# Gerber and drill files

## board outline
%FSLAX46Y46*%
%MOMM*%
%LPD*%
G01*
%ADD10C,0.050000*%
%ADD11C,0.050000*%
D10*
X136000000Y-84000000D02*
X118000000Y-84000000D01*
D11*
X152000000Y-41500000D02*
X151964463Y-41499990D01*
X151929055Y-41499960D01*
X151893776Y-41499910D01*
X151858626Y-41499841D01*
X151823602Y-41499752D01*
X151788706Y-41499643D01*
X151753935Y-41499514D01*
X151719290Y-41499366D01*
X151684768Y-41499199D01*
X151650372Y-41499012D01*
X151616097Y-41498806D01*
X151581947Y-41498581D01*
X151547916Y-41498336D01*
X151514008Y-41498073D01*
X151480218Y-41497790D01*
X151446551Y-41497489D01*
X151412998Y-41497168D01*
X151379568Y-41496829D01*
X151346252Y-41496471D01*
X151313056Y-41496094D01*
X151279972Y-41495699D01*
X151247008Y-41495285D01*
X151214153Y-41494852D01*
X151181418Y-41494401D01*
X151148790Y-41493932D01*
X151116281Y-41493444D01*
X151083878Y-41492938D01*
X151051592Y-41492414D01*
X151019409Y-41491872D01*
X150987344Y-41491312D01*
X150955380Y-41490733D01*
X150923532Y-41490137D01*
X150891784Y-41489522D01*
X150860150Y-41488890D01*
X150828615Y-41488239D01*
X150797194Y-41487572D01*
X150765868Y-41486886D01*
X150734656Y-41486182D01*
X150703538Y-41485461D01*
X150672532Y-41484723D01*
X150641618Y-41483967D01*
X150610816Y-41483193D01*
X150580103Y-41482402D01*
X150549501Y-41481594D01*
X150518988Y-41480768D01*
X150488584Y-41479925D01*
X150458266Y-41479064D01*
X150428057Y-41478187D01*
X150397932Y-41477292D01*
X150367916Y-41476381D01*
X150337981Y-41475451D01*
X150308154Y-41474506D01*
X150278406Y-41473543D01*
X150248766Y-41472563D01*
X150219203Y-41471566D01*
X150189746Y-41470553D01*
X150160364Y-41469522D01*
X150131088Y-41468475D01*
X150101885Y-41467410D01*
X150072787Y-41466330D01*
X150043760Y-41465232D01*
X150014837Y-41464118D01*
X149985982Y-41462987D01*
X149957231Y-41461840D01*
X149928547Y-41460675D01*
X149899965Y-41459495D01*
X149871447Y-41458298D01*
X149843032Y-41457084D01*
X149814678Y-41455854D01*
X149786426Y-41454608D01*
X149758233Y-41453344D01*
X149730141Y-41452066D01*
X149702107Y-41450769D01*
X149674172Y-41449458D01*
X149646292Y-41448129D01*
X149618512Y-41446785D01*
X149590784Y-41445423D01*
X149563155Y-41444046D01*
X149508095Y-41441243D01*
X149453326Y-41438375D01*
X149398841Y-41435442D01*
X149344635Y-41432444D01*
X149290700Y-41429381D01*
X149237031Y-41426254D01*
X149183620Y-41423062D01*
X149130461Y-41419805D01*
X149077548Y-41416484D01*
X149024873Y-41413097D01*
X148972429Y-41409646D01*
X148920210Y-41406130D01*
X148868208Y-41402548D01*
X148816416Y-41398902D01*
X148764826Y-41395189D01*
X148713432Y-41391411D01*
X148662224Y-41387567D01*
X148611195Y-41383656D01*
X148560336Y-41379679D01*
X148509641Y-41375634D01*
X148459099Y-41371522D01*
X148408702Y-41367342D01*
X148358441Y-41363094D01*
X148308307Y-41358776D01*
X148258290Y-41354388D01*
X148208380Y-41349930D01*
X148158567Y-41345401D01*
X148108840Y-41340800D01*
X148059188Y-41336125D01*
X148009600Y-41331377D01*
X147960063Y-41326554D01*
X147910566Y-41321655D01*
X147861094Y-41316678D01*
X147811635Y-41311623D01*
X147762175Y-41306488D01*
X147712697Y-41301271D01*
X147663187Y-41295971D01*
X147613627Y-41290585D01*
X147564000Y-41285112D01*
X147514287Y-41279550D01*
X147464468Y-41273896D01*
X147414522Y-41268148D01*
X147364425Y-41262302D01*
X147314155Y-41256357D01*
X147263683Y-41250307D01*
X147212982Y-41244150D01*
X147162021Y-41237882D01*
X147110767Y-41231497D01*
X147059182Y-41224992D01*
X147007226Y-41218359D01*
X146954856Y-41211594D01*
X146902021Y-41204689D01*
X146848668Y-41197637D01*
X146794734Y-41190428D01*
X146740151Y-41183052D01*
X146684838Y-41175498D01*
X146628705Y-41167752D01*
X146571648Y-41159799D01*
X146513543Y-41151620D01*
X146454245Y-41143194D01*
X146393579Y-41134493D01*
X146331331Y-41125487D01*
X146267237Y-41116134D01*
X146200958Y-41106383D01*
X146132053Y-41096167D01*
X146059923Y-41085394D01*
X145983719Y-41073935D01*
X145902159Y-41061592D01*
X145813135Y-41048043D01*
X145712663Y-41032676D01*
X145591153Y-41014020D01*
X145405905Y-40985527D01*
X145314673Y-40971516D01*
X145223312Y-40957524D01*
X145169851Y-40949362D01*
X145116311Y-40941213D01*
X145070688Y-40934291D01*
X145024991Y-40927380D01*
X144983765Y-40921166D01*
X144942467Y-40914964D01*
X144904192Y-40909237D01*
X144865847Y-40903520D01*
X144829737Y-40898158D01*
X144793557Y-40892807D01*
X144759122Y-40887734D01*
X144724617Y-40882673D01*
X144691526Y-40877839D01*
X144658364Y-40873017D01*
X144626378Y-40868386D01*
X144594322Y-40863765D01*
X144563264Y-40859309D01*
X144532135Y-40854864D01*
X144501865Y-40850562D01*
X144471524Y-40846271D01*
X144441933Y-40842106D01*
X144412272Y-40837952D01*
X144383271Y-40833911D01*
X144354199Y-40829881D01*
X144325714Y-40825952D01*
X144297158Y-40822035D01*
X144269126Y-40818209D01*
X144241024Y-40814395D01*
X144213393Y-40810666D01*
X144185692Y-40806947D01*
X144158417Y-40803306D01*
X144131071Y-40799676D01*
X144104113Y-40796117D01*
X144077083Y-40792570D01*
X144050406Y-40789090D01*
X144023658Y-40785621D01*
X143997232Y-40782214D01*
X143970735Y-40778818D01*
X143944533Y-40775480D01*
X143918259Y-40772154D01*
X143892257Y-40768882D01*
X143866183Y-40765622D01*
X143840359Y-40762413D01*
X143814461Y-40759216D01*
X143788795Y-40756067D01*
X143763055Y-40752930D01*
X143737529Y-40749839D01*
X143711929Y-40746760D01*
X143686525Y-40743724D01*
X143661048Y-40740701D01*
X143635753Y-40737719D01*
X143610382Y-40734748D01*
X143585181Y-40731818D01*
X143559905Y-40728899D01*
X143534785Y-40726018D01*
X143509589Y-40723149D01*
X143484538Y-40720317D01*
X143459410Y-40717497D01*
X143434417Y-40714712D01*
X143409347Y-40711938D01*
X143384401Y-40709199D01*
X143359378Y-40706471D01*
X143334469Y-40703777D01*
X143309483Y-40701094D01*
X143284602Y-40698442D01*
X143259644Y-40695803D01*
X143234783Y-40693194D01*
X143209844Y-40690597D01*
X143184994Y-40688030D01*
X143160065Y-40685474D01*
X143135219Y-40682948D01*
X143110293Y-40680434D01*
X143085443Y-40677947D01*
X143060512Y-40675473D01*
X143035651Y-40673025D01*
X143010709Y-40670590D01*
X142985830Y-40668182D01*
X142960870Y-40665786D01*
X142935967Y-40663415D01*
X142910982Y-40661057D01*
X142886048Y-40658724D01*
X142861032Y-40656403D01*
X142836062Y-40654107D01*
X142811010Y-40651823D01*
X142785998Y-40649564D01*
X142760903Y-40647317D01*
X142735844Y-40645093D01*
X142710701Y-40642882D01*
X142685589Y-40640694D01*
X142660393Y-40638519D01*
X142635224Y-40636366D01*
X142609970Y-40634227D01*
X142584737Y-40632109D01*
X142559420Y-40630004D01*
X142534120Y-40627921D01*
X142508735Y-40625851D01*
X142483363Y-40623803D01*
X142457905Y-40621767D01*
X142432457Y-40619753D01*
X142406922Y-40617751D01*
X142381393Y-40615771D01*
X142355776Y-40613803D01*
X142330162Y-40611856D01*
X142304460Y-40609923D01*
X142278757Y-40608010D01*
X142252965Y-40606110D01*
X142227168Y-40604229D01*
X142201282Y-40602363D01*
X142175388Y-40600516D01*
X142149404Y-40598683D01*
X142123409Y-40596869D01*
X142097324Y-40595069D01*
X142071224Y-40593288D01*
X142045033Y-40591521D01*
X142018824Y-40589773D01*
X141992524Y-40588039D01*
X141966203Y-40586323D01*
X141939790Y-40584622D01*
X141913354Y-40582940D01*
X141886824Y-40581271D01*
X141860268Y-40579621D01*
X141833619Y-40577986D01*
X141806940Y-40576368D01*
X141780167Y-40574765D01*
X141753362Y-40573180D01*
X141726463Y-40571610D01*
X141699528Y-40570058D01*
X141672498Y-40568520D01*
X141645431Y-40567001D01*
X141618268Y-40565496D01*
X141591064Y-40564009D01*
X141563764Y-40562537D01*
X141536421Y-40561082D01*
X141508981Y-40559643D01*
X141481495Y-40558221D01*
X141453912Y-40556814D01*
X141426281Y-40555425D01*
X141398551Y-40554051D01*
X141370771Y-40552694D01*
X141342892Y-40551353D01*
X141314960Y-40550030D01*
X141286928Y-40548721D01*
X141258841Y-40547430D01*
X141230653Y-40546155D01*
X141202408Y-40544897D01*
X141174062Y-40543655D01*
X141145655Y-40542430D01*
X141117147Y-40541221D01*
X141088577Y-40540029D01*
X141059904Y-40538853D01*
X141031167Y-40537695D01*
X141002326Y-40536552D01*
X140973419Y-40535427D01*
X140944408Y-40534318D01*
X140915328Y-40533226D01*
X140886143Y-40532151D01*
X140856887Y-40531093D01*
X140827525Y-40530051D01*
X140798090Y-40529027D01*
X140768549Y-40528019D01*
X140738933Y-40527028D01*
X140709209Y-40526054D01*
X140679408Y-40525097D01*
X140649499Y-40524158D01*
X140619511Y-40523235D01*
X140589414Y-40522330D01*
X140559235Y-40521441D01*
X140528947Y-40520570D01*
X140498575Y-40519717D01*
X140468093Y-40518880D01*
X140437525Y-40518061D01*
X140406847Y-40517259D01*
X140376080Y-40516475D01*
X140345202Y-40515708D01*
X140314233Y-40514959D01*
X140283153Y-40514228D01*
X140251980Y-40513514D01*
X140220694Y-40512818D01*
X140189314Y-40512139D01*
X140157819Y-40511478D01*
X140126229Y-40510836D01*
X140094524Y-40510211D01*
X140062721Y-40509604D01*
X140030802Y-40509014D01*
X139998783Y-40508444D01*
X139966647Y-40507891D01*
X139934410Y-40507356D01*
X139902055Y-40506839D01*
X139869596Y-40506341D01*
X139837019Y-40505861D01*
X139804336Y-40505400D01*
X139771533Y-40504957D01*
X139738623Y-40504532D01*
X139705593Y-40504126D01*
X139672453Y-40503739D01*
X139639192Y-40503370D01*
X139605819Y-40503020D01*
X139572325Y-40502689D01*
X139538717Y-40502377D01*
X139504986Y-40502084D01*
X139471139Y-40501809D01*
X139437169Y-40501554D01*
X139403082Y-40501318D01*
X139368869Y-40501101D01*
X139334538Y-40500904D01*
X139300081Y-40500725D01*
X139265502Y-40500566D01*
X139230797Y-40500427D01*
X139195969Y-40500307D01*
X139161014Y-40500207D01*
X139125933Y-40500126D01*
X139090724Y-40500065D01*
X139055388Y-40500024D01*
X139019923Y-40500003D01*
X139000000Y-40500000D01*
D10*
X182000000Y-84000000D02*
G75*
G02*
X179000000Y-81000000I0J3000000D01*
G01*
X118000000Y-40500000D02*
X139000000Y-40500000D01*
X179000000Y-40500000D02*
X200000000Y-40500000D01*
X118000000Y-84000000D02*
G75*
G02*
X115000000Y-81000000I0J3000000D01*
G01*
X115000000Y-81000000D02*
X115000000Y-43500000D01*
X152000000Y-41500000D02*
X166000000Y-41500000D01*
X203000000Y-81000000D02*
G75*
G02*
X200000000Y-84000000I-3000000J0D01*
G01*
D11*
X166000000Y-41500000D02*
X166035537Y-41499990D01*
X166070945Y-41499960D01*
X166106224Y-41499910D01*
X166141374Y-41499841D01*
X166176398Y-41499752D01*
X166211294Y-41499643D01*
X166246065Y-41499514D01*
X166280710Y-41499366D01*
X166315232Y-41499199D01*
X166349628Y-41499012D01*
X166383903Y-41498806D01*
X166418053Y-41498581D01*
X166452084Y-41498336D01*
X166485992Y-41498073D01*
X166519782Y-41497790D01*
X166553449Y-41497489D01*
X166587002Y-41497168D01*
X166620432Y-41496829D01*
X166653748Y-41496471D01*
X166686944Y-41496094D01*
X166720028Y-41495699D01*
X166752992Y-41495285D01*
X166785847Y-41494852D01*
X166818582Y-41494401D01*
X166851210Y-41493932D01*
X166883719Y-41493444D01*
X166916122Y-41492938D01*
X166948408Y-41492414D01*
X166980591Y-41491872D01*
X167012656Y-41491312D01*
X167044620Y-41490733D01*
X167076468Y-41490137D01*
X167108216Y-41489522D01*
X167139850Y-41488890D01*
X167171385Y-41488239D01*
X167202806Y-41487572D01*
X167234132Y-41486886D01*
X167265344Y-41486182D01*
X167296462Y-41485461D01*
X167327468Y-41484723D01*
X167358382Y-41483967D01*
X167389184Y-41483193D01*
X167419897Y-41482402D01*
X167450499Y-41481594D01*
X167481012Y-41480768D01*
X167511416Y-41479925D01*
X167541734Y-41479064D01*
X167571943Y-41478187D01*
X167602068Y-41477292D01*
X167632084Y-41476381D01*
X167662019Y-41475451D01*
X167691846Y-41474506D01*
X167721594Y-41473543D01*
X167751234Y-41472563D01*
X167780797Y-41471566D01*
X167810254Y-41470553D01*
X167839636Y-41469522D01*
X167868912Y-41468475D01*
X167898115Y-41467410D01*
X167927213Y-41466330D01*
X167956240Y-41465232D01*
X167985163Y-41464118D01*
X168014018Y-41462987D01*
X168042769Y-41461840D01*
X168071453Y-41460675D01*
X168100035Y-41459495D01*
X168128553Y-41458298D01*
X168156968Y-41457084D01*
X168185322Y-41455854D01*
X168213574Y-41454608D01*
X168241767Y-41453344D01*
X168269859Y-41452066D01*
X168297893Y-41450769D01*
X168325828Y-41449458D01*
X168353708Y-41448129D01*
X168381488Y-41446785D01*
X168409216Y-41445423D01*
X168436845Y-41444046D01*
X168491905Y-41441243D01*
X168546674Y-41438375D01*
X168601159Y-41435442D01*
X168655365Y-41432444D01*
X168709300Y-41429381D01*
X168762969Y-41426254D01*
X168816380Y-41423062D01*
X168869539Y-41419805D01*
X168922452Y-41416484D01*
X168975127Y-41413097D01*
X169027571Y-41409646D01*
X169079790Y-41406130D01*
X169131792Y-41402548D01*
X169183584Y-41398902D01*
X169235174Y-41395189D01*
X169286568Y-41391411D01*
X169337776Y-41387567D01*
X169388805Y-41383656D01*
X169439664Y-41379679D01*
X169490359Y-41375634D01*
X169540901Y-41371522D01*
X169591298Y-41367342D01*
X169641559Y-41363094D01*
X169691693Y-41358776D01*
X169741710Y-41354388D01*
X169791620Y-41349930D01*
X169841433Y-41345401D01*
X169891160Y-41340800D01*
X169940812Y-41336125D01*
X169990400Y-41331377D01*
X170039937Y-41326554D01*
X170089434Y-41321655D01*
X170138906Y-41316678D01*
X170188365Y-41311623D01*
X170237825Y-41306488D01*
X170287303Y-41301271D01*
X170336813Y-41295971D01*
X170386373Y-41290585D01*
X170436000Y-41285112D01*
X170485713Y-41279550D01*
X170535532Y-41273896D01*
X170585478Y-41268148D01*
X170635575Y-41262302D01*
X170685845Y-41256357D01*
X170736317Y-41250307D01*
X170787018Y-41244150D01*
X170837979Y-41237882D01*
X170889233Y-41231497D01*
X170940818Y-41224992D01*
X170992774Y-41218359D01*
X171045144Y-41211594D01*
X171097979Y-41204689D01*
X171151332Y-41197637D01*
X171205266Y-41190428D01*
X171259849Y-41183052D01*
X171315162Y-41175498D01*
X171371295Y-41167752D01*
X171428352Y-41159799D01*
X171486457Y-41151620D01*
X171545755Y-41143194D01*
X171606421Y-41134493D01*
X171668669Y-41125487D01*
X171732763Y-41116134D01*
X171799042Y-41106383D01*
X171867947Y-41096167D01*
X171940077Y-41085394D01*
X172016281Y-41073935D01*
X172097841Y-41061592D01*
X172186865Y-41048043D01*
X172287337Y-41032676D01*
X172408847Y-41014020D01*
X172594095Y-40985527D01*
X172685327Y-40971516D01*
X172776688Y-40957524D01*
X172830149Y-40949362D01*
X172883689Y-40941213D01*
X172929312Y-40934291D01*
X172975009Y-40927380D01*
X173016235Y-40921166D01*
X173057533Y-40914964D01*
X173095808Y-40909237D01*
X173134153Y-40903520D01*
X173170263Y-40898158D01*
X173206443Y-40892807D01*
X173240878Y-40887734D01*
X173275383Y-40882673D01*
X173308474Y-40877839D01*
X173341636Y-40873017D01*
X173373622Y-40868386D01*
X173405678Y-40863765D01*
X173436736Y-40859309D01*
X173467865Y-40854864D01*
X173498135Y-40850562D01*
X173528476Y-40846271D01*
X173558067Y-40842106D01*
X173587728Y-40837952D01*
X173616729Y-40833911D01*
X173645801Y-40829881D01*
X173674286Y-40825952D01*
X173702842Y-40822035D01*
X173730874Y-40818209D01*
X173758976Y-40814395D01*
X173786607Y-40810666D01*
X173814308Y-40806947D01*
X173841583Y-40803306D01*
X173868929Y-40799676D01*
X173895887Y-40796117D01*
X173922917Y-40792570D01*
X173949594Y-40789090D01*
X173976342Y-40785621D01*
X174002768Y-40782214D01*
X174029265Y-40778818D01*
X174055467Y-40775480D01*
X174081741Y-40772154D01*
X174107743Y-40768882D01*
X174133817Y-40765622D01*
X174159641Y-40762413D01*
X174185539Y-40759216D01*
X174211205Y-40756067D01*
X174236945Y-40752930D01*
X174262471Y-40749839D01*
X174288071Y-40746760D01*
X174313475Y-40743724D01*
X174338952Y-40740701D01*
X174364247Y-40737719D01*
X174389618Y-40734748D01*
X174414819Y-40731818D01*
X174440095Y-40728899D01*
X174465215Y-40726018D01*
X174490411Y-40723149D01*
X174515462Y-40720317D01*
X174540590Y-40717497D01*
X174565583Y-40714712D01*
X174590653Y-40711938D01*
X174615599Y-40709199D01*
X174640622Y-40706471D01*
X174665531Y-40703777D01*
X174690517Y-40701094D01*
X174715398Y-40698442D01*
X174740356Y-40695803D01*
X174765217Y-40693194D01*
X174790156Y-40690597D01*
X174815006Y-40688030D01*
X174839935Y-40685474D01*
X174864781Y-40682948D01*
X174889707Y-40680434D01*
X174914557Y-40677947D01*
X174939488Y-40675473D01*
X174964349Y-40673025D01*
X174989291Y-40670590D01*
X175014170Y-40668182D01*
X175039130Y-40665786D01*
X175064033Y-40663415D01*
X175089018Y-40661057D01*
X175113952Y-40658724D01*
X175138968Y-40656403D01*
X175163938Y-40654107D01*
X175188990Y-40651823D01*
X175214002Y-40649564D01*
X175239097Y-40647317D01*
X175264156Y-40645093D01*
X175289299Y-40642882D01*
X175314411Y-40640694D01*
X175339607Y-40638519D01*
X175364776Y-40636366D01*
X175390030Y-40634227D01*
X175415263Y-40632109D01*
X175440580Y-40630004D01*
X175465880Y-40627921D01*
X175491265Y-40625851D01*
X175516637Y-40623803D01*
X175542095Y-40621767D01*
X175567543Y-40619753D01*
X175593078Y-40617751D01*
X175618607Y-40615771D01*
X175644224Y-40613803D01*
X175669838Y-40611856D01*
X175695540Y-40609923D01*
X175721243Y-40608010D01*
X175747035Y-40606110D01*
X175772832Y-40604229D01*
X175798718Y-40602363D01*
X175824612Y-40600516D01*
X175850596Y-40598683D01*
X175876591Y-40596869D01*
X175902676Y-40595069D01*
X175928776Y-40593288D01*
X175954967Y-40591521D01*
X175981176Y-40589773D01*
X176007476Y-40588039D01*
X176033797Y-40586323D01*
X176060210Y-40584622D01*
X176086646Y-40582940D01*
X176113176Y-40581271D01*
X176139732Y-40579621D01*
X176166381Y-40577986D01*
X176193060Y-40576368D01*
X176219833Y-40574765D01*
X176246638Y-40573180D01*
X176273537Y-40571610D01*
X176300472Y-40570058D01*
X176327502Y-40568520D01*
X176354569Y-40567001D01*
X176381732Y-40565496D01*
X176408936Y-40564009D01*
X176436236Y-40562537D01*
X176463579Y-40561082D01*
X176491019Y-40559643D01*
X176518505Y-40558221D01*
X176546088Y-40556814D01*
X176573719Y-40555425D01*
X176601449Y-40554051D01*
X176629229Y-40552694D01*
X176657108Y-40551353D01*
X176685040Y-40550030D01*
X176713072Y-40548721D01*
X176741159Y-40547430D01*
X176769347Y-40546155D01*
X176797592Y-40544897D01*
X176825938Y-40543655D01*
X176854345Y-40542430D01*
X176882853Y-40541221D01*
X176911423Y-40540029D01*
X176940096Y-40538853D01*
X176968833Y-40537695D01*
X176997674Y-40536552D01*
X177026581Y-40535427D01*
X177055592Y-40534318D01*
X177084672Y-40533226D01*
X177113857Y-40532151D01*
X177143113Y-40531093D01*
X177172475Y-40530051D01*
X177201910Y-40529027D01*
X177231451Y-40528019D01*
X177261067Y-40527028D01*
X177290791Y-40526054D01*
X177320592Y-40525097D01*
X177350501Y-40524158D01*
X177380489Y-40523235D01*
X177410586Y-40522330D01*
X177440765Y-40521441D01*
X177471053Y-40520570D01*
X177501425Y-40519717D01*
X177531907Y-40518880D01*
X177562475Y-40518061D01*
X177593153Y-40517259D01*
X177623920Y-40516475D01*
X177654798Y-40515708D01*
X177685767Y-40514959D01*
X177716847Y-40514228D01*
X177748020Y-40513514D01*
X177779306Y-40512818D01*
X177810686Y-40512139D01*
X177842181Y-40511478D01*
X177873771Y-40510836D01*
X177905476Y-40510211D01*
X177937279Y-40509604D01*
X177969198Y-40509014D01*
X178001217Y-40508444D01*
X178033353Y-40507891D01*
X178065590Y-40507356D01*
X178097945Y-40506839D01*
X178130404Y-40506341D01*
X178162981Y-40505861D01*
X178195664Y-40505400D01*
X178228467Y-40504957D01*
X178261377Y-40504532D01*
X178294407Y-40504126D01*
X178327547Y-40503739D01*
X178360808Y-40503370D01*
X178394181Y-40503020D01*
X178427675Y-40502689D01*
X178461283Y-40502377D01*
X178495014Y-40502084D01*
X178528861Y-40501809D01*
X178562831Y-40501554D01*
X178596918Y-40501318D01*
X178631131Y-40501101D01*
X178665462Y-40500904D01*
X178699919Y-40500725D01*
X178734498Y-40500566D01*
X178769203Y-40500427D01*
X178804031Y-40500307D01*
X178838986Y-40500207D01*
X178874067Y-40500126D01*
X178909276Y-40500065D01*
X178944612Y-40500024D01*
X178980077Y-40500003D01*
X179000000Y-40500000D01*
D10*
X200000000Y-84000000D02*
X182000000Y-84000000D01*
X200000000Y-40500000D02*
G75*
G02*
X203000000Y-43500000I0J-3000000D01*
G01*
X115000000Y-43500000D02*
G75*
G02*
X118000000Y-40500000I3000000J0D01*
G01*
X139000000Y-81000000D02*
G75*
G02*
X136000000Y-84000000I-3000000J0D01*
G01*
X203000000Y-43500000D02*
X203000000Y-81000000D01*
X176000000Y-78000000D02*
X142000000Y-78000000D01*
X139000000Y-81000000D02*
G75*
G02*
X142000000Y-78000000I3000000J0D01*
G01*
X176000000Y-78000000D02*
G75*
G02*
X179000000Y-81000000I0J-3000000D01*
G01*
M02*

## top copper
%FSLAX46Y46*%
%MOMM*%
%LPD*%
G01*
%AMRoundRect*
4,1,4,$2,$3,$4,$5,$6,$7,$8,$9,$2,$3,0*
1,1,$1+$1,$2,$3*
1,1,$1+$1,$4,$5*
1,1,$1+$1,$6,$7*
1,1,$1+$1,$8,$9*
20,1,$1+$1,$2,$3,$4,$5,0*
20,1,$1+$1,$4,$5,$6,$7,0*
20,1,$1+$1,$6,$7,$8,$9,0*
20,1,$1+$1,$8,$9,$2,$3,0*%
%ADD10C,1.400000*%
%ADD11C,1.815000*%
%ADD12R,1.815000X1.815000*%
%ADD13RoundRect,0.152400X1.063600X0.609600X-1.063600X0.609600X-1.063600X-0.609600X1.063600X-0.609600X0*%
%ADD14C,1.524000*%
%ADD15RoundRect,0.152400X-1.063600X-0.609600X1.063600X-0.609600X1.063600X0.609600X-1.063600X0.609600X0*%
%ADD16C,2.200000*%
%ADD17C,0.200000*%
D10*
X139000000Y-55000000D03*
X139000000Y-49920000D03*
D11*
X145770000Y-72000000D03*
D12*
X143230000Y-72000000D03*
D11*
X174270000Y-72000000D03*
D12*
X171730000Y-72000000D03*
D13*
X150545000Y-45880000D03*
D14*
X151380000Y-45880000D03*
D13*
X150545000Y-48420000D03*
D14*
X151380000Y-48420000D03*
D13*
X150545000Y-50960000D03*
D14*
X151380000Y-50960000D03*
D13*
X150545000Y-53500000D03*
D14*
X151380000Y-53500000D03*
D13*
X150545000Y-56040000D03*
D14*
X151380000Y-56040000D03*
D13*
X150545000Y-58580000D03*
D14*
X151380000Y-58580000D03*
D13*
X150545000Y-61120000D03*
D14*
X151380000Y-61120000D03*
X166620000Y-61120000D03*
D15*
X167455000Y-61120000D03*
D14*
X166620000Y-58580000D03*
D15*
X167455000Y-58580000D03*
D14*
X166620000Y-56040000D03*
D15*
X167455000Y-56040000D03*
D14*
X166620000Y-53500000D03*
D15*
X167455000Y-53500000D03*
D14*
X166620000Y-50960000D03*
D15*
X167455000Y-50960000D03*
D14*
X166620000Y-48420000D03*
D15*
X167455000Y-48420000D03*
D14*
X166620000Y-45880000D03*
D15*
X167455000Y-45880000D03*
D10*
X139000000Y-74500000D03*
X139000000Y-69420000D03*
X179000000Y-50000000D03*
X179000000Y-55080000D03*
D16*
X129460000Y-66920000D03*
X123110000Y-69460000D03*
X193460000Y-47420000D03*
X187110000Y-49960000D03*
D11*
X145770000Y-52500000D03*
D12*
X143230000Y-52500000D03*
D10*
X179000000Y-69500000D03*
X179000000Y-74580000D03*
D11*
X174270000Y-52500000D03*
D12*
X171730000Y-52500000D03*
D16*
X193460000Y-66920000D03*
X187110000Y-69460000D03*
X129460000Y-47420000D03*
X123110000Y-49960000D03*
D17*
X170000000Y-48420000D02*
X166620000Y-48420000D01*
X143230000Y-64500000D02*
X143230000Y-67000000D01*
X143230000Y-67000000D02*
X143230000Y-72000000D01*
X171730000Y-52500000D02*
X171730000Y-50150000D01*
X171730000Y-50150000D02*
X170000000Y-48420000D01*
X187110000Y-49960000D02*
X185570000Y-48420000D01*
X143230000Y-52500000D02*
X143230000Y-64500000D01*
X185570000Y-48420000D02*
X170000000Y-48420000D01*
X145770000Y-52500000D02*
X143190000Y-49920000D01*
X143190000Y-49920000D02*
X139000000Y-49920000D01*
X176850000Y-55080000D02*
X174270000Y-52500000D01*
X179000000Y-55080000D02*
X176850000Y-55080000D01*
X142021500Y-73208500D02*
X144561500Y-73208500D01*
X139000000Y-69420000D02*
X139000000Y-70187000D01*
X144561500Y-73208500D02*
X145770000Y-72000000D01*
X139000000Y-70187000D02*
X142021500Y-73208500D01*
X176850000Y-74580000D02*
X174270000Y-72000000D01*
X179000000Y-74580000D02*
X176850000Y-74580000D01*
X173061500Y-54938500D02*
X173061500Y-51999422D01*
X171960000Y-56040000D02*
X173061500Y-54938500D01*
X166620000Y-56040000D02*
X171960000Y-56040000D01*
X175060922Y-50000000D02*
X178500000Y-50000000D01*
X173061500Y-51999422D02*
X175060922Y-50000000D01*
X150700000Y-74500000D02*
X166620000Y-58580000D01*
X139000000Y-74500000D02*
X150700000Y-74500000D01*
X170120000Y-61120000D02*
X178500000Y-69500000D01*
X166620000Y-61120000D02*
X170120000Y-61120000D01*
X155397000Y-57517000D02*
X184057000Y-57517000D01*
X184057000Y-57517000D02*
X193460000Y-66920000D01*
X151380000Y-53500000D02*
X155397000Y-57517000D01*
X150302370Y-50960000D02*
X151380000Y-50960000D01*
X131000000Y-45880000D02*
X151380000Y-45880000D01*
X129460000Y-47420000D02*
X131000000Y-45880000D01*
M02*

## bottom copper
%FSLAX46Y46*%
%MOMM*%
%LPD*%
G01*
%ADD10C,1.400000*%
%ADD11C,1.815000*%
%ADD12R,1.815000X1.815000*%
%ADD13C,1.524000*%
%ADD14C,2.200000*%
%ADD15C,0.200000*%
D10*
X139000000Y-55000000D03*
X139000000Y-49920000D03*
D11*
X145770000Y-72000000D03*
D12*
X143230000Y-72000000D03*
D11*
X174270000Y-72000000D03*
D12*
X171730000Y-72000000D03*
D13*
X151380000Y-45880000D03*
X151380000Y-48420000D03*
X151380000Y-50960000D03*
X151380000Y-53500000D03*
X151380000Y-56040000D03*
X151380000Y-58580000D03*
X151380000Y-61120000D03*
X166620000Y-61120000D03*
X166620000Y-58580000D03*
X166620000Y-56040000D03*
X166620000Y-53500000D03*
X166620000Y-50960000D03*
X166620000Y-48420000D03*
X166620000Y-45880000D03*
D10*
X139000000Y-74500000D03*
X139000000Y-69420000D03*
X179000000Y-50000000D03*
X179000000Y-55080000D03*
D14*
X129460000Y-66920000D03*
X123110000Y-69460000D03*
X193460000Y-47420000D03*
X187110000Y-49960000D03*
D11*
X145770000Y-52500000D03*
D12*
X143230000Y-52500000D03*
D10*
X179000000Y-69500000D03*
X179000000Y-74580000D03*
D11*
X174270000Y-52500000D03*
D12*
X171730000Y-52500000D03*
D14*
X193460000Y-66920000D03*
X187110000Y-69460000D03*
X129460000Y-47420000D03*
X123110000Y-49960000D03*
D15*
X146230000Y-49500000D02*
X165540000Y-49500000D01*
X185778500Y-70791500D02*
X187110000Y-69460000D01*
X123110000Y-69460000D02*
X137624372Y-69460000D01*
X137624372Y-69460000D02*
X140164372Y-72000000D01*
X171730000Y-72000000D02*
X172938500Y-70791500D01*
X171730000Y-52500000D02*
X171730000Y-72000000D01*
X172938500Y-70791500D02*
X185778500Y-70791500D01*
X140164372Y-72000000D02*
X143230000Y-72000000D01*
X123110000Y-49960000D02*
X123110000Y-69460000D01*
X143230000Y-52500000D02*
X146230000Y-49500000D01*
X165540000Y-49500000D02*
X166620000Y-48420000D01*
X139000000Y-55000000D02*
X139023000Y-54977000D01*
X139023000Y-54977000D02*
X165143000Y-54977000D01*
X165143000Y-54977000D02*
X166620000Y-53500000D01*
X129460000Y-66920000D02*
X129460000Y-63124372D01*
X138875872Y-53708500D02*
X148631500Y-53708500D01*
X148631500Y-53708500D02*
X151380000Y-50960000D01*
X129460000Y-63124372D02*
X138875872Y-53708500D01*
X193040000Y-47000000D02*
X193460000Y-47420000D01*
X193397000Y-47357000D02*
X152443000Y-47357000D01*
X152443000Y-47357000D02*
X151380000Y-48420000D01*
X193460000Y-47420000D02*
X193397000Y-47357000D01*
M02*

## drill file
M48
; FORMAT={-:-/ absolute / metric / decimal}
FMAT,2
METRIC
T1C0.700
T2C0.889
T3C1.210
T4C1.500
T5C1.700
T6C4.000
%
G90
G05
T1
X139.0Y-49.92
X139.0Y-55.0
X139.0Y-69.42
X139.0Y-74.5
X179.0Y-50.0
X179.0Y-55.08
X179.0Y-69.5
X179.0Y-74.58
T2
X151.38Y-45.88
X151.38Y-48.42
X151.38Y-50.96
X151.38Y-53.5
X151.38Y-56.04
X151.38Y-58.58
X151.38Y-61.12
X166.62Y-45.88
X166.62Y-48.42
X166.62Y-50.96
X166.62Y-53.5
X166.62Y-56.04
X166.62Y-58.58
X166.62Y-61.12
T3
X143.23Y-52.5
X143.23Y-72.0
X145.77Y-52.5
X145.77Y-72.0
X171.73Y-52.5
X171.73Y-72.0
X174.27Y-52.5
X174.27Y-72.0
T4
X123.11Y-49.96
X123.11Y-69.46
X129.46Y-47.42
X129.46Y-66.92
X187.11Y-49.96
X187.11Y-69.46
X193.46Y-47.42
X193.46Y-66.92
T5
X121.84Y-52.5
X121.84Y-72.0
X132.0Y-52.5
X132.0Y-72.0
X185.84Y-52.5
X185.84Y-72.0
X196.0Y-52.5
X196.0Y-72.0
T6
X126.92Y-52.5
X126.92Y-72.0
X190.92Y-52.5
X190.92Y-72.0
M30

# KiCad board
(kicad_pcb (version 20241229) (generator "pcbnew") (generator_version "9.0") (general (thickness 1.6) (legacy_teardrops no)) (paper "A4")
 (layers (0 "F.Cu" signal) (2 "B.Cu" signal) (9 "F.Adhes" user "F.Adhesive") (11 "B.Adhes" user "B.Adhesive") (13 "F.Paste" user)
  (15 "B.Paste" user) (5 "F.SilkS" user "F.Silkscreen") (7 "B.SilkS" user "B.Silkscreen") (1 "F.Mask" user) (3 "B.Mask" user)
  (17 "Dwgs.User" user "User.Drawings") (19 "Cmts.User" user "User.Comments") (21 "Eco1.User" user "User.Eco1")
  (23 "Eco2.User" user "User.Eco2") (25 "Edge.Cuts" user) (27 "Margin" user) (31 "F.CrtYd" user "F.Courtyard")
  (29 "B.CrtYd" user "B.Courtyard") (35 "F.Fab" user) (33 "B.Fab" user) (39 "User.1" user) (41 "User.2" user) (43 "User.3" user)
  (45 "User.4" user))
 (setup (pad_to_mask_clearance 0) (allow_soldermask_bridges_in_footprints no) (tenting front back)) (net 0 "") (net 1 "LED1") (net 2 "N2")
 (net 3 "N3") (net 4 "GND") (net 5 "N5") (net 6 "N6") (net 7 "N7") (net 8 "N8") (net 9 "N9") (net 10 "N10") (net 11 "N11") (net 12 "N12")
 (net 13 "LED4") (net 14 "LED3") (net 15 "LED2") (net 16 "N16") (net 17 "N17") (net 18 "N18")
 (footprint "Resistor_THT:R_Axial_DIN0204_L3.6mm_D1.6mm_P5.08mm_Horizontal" (layer "F.Cu") (at 139 55 90)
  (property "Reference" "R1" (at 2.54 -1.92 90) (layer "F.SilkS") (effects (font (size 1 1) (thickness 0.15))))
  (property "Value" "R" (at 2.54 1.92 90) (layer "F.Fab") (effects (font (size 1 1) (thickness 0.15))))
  (pad "1" thru_hole circle (at 0 0 90) (size 1.4 1.4) (drill 0.7) (layers "*.Cu" "*.Mask") (remove_unused_layers no) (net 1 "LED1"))
  (pad "2" thru_hole circle (at 5.08 0 90) (size 1.4 1.4) (drill 0.7) (layers "*.Cu" "*.Mask") (remove_unused_layers no) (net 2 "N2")))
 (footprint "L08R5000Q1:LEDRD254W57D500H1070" (layer "F.Cu") (at 144.5 72)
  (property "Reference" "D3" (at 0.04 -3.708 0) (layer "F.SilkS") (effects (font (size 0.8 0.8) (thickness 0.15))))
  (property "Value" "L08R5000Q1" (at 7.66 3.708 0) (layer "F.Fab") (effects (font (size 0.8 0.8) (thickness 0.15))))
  (pad "A" thru_hole circle (at 1.27 0) (size 1.815 1.815) (drill 1.21) (layers "*.Cu" "*.Mask") (remove_unused_layers no) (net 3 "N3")
   (solder_mask_margin 0.102))
  (pad "C" thru_hole rect (at -1.27 0) (size 1.815 1.815) (drill 1.21) (layers "*.Cu" "*.Mask") (remove_unused_layers no) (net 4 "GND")
   (solder_mask_margin 0.102)))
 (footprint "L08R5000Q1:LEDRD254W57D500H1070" (layer "F.Cu") (at 173 72)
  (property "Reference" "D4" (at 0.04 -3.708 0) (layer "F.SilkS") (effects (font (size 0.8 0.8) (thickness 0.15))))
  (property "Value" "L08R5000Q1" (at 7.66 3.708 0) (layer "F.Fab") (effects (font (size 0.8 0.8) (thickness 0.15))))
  (pad "A" thru_hole circle (at 1.27 0) (size 1.815 1.815) (drill 1.21) (layers "*.Cu" "*.Mask") (remove_unused_layers no) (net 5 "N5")
   (solder_mask_margin 0.102))
  (pad "C" thru_hole rect (at -1.27 0) (size 1.815 1.815) (drill 1.21) (layers "*.Cu" "*.Mask") (remove_unused_layers no) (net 4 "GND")
   (solder_mask_margin 0.102)))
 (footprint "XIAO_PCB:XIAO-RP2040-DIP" (layer "F.Cu") (at 159 53.5)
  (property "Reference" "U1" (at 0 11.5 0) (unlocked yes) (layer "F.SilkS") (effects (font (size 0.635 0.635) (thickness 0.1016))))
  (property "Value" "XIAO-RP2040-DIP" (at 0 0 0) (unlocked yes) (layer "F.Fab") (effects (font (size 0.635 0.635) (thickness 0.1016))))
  (pad "1" smd roundrect (at -8.455 -7.62 180) (size 2.432 1.524) (layers "F.Cu" "F.Mask") (roundrect_rratio 0.1) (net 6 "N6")
   (thermal_bridge_angle 45))
  (pad "1" thru_hole circle (at -7.62 -7.62 180) (size 1.524 1.524) (drill 0.889) (layers "*.Cu" "*.Mask") (remove_unused_layers no)
   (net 6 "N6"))
  (pad "2" smd roundrect (at -8.455 -5.08 180) (size 2.432 1.524) (layers "F.Cu" "F.Mask") (roundrect_rratio 0.1) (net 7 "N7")
   (thermal_bridge_angle 45))
  (pad "2" thru_hole circle (at -7.62 -5.08 180) (size 1.524 1.524) (drill 0.889) (layers "*.Cu" "*.Mask") (remove_unused_layers no)
   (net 7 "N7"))
  (pad "3" smd roundrect (at -8.455 -2.54 180) (size 2.432 1.524) (layers "F.Cu" "F.Mask") (roundrect_rratio 0.1) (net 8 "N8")
   (thermal_bridge_angle 45))
  (pad "3" thru_hole circle (at -7.62 -2.54 180) (size 1.524 1.524) (drill 0.889) (layers "*.Cu" "*.Mask") (remove_unused_layers no)
   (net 8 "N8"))
  (pad "4" smd roundrect (at -8.455 0 180) (size 2.432 1.524) (layers "F.Cu" "F.Mask") (roundrect_rratio 0.1) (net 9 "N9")
   (thermal_bridge_angle 45))
  (pad "4" thru_hole circle (at -7.62 0 180) (size 1.524 1.524) (drill 0.889) (layers "*.Cu" "*.Mask") (remove_unused_layers no)
   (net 9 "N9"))
  (pad "5" smd roundrect (at -8.455 2.54 180) (size 2.432 1.524) (layers "F.Cu" "F.Mask") (roundrect_rratio 0.1) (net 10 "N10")
   (thermal_bridge_angle 45))
  (pad "5" thru_hole circle (at -7.62 2.54 180) (size 1.524 1.524) (drill 0.889) (layers "*.Cu" "*.Mask") (remove_unused_layers no)
   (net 10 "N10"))
  (pad "6" smd roundrect (at -8.455 5.08 180) (size 2.432 1.524) (layers "F.Cu" "F.Mask") (roundrect_rratio 0.1) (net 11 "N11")
   (thermal_bridge_angle 45))
  (pad "6" thru_hole circle (at -7.62 5.08 180) (size 1.524 1.524) (drill 0.889) (layers "*.Cu" "*.Mask") (remove_unused_layers no)
   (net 11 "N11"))
  (pad "7" smd roundrect (at -8.455 7.62 180) (size 2.432 1.524) (layers "F.Cu" "F.Mask") (roundrect_rratio 0.1) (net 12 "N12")
   (thermal_bridge_angle 45))
  (pad "7" thru_hole circle (at -7.62 7.62 180) (size 1.524 1.524) (drill 0.889) (layers "*.Cu" "*.Mask") (remove_unused_layers no)
   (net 12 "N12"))
  (pad "8" thru_hole circle (at 7.62 7.62) (size 1.524 1.524) (drill 0.889) (layers "*.Cu" "*.Mask") (remove_unused_layers no)
   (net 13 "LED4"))
  (pad "8" smd roundrect (at 8.455 7.62) (size 2.432 1.524) (layers "F.Cu" "F.Mask") (roundrect_rratio 0.1) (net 13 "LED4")
   (thermal_bridge_angle 45))
  (pad "9" thru_hole circle (at 7.62 5.08) (size 1.524 1.524) (drill 0.889) (layers "*.Cu" "*.Mask") (remove_unused_layers no)
   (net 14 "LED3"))
  (pad "9" smd roundrect (at 8.455 5.08) (size 2.432 1.524) (layers "F.Cu" "F.Mask") (roundrect_rratio 0.1) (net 14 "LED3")
   (thermal_bridge_angle 45))
  (pad "10" thru_hole circle (at 7.62 2.54) (size 1.524 1.524) (drill 0.889) (layers "*.Cu" "*.Mask") (remove_unused_layers no)
   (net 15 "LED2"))
  (pad "10" smd roundrect (at 8.455 2.54) (size 2.432 1.524) (layers "F.Cu" "F.Mask") (roundrect_rratio 0.1) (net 15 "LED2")
   (thermal_bridge_angle 45))
  (pad "11" thru_hole circle (at 7.62 0) (size 1.524 1.524) (drill 0.889) (layers "*.Cu" "*.Mask") (remove_unused_layers no) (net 1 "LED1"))
  (pad "11" smd roundrect (at 8.455 0) (size 2.432 1.524) (layers "F.Cu" "F.Mask") (roundrect_rratio 0.1) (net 1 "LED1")
   (thermal_bridge_angle 45))
  (pad "12" thru_hole circle (at 7.62 -2.54) (size 1.524 1.524) (drill 0.889) (layers "*.Cu" "*.Mask") (remove_unused_layers no)
   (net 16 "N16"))
  (pad "12" smd roundrect (at 8.455 -2.54) (size 2.432 1.524) (layers "F.Cu" "F.Mask") (roundrect_rratio 0.1) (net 16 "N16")
   (thermal_bridge_angle 45))
  (pad "13" thru_hole circle (at 7.62 -5.08) (size 1.524 1.524) (drill 0.889) (layers "*.Cu" "*.Mask") (remove_unused_layers no)
   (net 4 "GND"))
  (pad "13" smd roundrect (at 8.455 -5.08) (size 2.432 1.524) (layers "F.Cu" "F.Mask") (roundrect_rratio 0.1) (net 4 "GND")
   (thermal_bridge_angle 45))
  (pad "14" thru_hole circle (at 7.62 -7.62) (size 1.524 1.524) (drill 0.889) (layers "*.Cu" "*.Mask") (remove_unused_layers no)
   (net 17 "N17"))
  (pad "14" smd roundrect (at 8.455 -7.62) (size 2.432 1.524) (layers "F.Cu" "F.Mask") (roundrect_rratio 0.1) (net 17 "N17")
   (thermal_bridge_angle 45)))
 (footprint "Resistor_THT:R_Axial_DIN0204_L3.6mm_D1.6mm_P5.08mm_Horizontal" (layer "F.Cu") (at 139 74.5 90)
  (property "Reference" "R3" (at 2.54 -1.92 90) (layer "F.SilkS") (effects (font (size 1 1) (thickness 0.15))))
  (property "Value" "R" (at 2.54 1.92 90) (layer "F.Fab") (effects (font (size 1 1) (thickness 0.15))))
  (pad "1" thru_hole circle (at 0 0 90) (size 1.4 1.4) (drill 0.7) (layers "*.Cu" "*.Mask") (remove_unused_layers no) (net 14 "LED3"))
  (pad "2" thru_hole circle (at 5.08 0 90) (size 1.4 1.4) (drill 0.7) (layers "*.Cu" "*.Mask") (remove_unused_layers no) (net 3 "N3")))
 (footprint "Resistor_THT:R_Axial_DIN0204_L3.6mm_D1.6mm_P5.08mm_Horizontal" (layer "F.Cu") (at 179 50 -90)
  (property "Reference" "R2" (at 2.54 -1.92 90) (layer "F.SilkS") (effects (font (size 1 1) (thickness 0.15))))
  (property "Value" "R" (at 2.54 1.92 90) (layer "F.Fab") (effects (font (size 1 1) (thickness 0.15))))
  (pad "1" thru_hole circle (at 0 0 270) (size 1.4 1.4) (drill 0.7) (layers "*.Cu" "*.Mask") (remove_unused_layers no) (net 15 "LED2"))
  (pad "2" thru_hole circle (at 5.08 0 270) (size 1.4 1.4) (drill 0.7) (layers "*.Cu" "*.Mask") (remove_unused_layers no) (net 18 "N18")))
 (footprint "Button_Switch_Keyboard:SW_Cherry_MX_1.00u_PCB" (layer "F.Cu") (at 129.46 66.92)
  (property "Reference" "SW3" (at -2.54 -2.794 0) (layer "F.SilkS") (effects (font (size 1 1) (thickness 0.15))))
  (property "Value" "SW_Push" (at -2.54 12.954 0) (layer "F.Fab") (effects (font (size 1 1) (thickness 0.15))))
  (pad "" np_thru_hole circle (at -7.62 5.08) (size 1.7 1.7) (drill 1.7) (layers "*.Cu" "*.Mask"))
  (pad "" np_thru_hole circle (at -2.54 5.08) (size 4 4) (drill 4) (layers "*.Cu" "*.Mask"))
  (pad "" np_thru_hole circle (at 2.54 5.08) (size 1.7 1.7) (drill 1.7) (layers "*.Cu" "*.Mask"))
  (pad "1" thru_hole circle (at 0 0) (size 2.2 2.2) (drill 1.5) (layers "*.Cu" "*.Mask") (remove_unused_layers no) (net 8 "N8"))
  (pad "2" thru_hole circle (at -6.35 2.54) (size 2.2 2.2) (drill 1.5) (layers "*.Cu" "*.Mask") (remove_unused_layers no) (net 4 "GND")))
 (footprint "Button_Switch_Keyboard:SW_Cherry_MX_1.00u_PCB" (layer "F.Cu") (at 193.46 47.42)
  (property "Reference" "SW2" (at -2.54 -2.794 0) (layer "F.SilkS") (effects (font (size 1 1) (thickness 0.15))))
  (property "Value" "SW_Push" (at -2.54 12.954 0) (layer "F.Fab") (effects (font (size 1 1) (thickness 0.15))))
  (pad "" np_thru_hole circle (at -7.62 5.08) (size 1.7 1.7) (drill 1.7) (layers "*.Cu" "*.Mask"))
  (pad "" np_thru_hole circle (at -2.54 5.08) (size 4 4) (drill 4) (layers "*.Cu" "*.Mask"))
  (pad "" np_thru_hole circle (at 2.54 5.08) (size 1.7 1.7) (drill 1.7) (layers "*.Cu" "*.Mask"))
  (pad "1" thru_hole circle (at 0 0) (size 2.2 2.2) (drill 1.5) (layers "*.Cu" "*.Mask") (remove_unused_layers no) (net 7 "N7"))
  (pad "2" thru_hole circle (at -6.35 2.54) (size 2.2 2.2) (drill 1.5) (layers "*.Cu" "*.Mask") (remove_unused_layers no) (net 4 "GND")))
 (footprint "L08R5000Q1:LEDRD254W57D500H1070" (layer "F.Cu") (at 144.5 52.5)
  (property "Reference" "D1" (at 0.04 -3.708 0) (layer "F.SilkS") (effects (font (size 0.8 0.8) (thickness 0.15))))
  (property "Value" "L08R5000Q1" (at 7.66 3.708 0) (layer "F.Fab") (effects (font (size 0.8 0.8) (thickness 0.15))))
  (pad "A" thru_hole circle (at 1.27 0) (size 1.815 1.815) (drill 1.21) (layers "*.Cu" "*.Mask") (remove_unused_layers no) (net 2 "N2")
   (solder_mask_margin 0.102))
  (pad "C" thru_hole rect (at -1.27 0) (size 1.815 1.815) (drill 1.21) (layers "*.Cu" "*.Mask") (remove_unused_layers no) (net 4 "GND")
   (solder_mask_margin 0.102)))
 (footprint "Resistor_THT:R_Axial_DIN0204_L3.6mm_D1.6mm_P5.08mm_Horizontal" (layer "F.Cu") (at 179 69.5 -90)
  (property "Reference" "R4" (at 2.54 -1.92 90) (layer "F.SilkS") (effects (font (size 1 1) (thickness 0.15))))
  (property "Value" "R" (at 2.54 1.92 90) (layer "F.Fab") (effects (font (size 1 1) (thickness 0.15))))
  (pad "1" thru_hole circle (at 0 0 270) (size 1.4 1.4) (drill 0.7) (layers "*.Cu" "*.Mask") (remove_unused_layers no) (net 13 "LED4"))
  (pad "2" thru_hole circle (at 5.08 0 270) (size 1.4 1.4) (drill 0.7) (layers "*.Cu" "*.Mask") (remove_unused_layers no) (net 5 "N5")))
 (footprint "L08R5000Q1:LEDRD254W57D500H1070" (layer "F.Cu") (at 173 52.5)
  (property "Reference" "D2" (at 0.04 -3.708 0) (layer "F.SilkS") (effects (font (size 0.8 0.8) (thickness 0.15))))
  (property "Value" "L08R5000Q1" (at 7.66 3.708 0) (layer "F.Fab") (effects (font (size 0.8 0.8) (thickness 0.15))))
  (pad "A" thru_hole circle (at 1.27 0) (size 1.815 1.815) (drill 1.21) (layers "*.Cu" "*.Mask") (remove_unused_layers no) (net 18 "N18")
   (solder_mask_margin 0.102))
  (pad "C" thru_hole rect (at -1.27 0) (size 1.815 1.815) (drill 1.21) (layers "*.Cu" "*.Mask") (remove_unused_layers no) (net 4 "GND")
   (solder_mask_margin 0.102)))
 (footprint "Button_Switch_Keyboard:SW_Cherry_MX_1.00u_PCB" (layer "F.Cu") (at 193.46 66.92)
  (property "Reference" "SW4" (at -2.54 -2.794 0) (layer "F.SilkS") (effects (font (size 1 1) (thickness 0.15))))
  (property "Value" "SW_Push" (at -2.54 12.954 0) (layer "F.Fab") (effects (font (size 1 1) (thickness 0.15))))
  (pad "" np_thru_hole circle (at -7.62 5.08) (size 1.7 1.7) (drill 1.7) (layers "*.Cu" "*.Mask"))
  (pad "" np_thru_hole circle (at -2.54 5.08) (size 4 4) (drill 4) (layers "*.Cu" "*.Mask"))
  (pad "" np_thru_hole circle (at 2.54 5.08) (size 1.7 1.7) (drill 1.7) (layers "*.Cu" "*.Mask"))
  (pad "1" thru_hole circle (at 0 0) (size 2.2 2.2) (drill 1.5) (layers "*.Cu" "*.Mask") (remove_unused_layers no) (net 9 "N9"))
  (pad "2" thru_hole circle (at -6.35 2.54) (size 2.2 2.2) (drill 1.5) (layers "*.Cu" "*.Mask") (remove_unused_layers no) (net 4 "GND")))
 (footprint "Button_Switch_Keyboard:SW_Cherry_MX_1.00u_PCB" (layer "F.Cu") (at 129.46 47.42)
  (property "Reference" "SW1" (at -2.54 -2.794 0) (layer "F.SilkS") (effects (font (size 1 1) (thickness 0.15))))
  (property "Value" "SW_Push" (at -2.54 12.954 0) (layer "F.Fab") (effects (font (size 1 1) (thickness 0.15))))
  (pad "" np_thru_hole circle (at -7.62 5.08) (size 1.7 1.7) (drill 1.7) (layers "*.Cu" "*.Mask"))
  (pad "" np_thru_hole circle (at -2.54 5.08) (size 4 4) (drill 4) (layers "*.Cu" "*.Mask"))
  (pad "" np_thru_hole circle (at 2.54 5.08) (size 1.7 1.7) (drill 1.7) (layers "*.Cu" "*.Mask"))
  (pad "1" thru_hole circle (at 0 0) (size 2.2 2.2) (drill 1.5) (layers "*.Cu" "*.Mask") (remove_unused_layers no) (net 6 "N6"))
  (pad "2" thru_hole circle (at -6.35 2.54) (size 2.2 2.2) (drill 1.5) (layers "*.Cu" "*.Mask") (remove_unused_layers no) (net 4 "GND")))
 (gr_line (start 136 84) (end 118 84) (stroke (width 0.05) (type default)) (layer "Edge.Cuts"))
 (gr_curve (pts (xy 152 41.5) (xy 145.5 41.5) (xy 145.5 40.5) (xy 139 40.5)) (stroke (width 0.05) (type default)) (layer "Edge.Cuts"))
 (gr_arc (start 182 84) (mid 179.87868 83.12132) (end 179 81) (stroke (width 0.05) (type default)) (layer "Edge.Cuts"))
 (gr_line (start 118 40.5) (end 139 40.5) (stroke (width 0.05) (type default)) (layer "Edge.Cuts"))
 (gr_line (start 179 40.5) (end 200 40.5) (stroke (width 0.05) (type default)) (layer "Edge.Cuts"))
 (gr_arc (start 118 84) (mid 115.87868 83.12132) (end 115 81) (stroke (width 0.05) (type default)) (layer "Edge.Cuts"))
 (gr_line (start 115 81) (end 115 43.5) (stroke (width 0.05) (type default)) (layer "Edge.Cuts"))
 (gr_line (start 152 41.5) (end 166 41.5) (stroke (width 0.05) (type default)) (layer "Edge.Cuts"))
 (gr_arc (start 203 81) (mid 202.12132 83.12132) (end 200 84) (stroke (width 0.05) (type default)) (layer "Edge.Cuts"))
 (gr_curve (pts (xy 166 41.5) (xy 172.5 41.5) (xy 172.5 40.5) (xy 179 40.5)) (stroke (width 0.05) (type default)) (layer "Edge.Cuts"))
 (gr_line (start 200 84) (end 182 84) (stroke (width 0.05) (type default)) (layer "Edge.Cuts"))
 (gr_arc (start 200 40.5) (mid 202.12132 41.37868) (end 203 43.5) (stroke (width 0.05) (type default)) (layer "Edge.Cuts"))
 (gr_arc (start 115 43.5) (mid 115.87868 41.37868) (end 118 40.5) (stroke (width 0.05) (type default)) (layer "Edge.Cuts"))
 (gr_arc (start 139 81) (mid 138.12132 83.12132) (end 136 84) (stroke (width 0.05) (type default)) (layer "Edge.Cuts"))
 (gr_line (start 203 43.5) (end 203 81) (stroke (width 0.05) (type default)) (layer "Edge.Cuts"))
 (gr_line (start 176 78) (end 142 78) (stroke (width 0.05) (type default)) (layer "Edge.Cuts"))
 (gr_arc (start 139 81) (mid 139.87868 78.87868) (end 142 78) (stroke (width 0.05) (type default)) (layer "Edge.Cuts"))
 (gr_arc (start 176 78) (mid 178.12132 78.87868) (end 179 81) (stroke (width 0.05) (type default)) (layer "Edge.Cuts"))
 (segment (start 170 48.42) (end 166.62 48.42) (width 0.2) (layer "F.Cu") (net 4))
 (segment (start 143.23 64.5) (end 143.23 67) (width 0.2) (layer "F.Cu") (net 4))
 (segment (start 143.23 67) (end 143.23 72) (width 0.2) (layer "F.Cu") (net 4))
 (segment (start 171.73 52.5) (end 171.73 50.15) (width 0.2) (layer "F.Cu") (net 4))
 (segment (start 171.73 50.15) (end 170 48.42) (width 0.2) (layer "F.Cu") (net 4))
 (segment (start 187.11 49.96) (end 185.57 48.42) (width 0.2) (layer "F.Cu") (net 4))
 (segment (start 143.23 52.5) (end 143.23 64.5) (width 0.2) (layer "F.Cu") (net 4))
 (segment (start 185.57 48.42) (end 170 48.42) (width 0.2) (layer "F.Cu") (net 4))
 (segment (start 146.23 49.5) (end 165.54 49.5) (width 0.2) (layer "B.Cu") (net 4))
 (segment (start 185.7785 70.7915) (end 187.11 69.46) (width 0.2) (layer "B.Cu") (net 4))
 (segment (start 123.11 69.46) (end 137.624372 69.46) (width 0.2) (layer "B.Cu") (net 4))
 (segment (start 137.624372 69.46) (end 140.164372 72) (width 0.2) (layer "B.Cu") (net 4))
 (segment (start 171.73 72) (end 172.9385 70.7915) (width 0.2) (layer "B.Cu") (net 4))
 (segment (start 171.73 52.5) (end 171.73 72) (width 0.2) (layer "B.Cu") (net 4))
 (segment (start 172.9385 70.7915) (end 185.7785 70.7915) (width 0.2) (layer "B.Cu") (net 4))
 (segment (start 140.164372 72) (end 143.23 72) (width 0.2) (layer "B.Cu") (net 4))
 (segment (start 123.11 49.96) (end 123.11 69.46) (width 0.2) (layer "B.Cu") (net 4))
 (segment (start 143.23 52.5) (end 146.23 49.5) (width 0.2) (layer "B.Cu") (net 4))
 (segment (start 165.54 49.5) (end 166.62 48.42) (width 0.2) (layer "B.Cu") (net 4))
 (segment (start 145.77 52.5) (end 143.19 49.92) (width 0.2) (layer "F.Cu") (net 2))
 (segment (start 143.19 49.92) (end 139 49.92) (width 0.2) (layer "F.Cu") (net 2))
 (segment (start 176.85 55.08) (end 174.27 52.5) (width 0.2) (layer "F.Cu") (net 18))
 (segment (start 179 55.08) (end 176.85 55.08) (width 0.2) (layer "F.Cu") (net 18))
 (segment (start 142.0215 73.2085) (end 144.5615 73.2085) (width 0.2) (layer "F.Cu") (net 3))
 (segment (start 139 69.42) (end 139 70.187) (width 0.2) (layer "F.Cu") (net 3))
 (segment (start 144.5615 73.2085) (end 145.77 72) (width 0.2) (layer "F.Cu") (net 3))
 (segment (start 139 70.187) (end 142.0215 73.2085) (width 0.2) (layer "F.Cu") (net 3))
 (segment (start 176.85 74.58) (end 174.27 72) (width 0.2) (layer "F.Cu") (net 5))
 (segment (start 179 74.58) (end 176.85 74.58) (width 0.2) (layer "F.Cu") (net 5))
 (segment (start 139 55) (end 139.023 54.977) (width 0.2) (layer "B.Cu") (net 1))
 (segment (start 139.023 54.977) (end 165.143 54.977) (width 0.2) (layer "B.Cu") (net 1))
 (segment (start 165.143 54.977) (end 166.62 53.5) (width 0.2) (layer "B.Cu") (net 1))
 (segment (start 173.0615 54.9385) (end 173.0615 51.999422) (width 0.2) (layer "F.Cu") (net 15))
 (segment (start 171.96 56.04) (end 173.0615 54.9385) (width 0.2) (layer "F.Cu") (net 15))
 (segment (start 166.62 56.04) (end 171.96 56.04) (width 0.2) (layer "F.Cu") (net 15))
 (segment (start 175.060922 50) (end 178.5 50) (width 0.2) (layer "F.Cu") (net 15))
 (segment (start 173.0615 51.999422) (end 175.060922 50) (width 0.2) (layer "F.Cu") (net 15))
 (segment (start 150.7 74.5) (end 166.62 58.58) (width 0.2) (layer "F.Cu") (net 14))
 (segment (start 139 74.5) (end 150.7 74.5) (width 0.2) (layer "F.Cu") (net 14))
 (segment (start 170.12 61.12) (end 178.5 69.5) (width 0.2) (layer "F.Cu") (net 13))
 (segment (start 166.62 61.12) (end 170.12 61.12) (width 0.2) (layer "F.Cu") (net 13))
 (segment (start 155.397 57.517) (end 184.057 57.517) (width 0.2) (layer "F.Cu") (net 9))
 (segment (start 184.057 57.517) (end 193.46 66.92) (width 0.2) (layer "F.Cu") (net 9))
 (segment (start 151.38 53.5) (end 155.397 57.517) (width 0.2) (layer "F.Cu") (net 9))
 (segment (start 150.30237 50.96) (end 151.38 50.96) (width 0.2) (layer "F.Cu") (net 8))
 (segment (start 129.46 66.92) (end 129.46 63.124372) (width 0.2) (layer "B.Cu") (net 8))
 (segment (start 138.875872 53.7085) (end 148.6315 53.7085) (width 0.2) (layer "B.Cu") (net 8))
 (segment (start 148.6315 53.7085) (end 151.38 50.96) (width 0.2) (layer "B.Cu") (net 8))
 (segment (start 129.46 63.124372) (end 138.875872 53.7085) (width 0.2) (layer "B.Cu") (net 8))
 (segment (start 193.04 47) (end 193.46 47.42) (width 0.2) (layer "B.Cu") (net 7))
 (segment (start 193.397 47.357) (end 152.443 47.357) (width 0.2) (layer "B.Cu") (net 7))
 (segment (start 152.443 47.357) (end 151.38 48.42) (width 0.2) (layer "B.Cu") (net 7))
 (segment (start 193.46 47.42) (end 193.397 47.357) (width 0.2) (layer "B.Cu") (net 7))
 (segment (start 131 45.88) (end 151.38 45.88) (width 0.2) (layer "F.Cu") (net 6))
 (segment (start 129.46 47.42) (end 131 45.88) (width 0.2) (layer "F.Cu") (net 6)))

